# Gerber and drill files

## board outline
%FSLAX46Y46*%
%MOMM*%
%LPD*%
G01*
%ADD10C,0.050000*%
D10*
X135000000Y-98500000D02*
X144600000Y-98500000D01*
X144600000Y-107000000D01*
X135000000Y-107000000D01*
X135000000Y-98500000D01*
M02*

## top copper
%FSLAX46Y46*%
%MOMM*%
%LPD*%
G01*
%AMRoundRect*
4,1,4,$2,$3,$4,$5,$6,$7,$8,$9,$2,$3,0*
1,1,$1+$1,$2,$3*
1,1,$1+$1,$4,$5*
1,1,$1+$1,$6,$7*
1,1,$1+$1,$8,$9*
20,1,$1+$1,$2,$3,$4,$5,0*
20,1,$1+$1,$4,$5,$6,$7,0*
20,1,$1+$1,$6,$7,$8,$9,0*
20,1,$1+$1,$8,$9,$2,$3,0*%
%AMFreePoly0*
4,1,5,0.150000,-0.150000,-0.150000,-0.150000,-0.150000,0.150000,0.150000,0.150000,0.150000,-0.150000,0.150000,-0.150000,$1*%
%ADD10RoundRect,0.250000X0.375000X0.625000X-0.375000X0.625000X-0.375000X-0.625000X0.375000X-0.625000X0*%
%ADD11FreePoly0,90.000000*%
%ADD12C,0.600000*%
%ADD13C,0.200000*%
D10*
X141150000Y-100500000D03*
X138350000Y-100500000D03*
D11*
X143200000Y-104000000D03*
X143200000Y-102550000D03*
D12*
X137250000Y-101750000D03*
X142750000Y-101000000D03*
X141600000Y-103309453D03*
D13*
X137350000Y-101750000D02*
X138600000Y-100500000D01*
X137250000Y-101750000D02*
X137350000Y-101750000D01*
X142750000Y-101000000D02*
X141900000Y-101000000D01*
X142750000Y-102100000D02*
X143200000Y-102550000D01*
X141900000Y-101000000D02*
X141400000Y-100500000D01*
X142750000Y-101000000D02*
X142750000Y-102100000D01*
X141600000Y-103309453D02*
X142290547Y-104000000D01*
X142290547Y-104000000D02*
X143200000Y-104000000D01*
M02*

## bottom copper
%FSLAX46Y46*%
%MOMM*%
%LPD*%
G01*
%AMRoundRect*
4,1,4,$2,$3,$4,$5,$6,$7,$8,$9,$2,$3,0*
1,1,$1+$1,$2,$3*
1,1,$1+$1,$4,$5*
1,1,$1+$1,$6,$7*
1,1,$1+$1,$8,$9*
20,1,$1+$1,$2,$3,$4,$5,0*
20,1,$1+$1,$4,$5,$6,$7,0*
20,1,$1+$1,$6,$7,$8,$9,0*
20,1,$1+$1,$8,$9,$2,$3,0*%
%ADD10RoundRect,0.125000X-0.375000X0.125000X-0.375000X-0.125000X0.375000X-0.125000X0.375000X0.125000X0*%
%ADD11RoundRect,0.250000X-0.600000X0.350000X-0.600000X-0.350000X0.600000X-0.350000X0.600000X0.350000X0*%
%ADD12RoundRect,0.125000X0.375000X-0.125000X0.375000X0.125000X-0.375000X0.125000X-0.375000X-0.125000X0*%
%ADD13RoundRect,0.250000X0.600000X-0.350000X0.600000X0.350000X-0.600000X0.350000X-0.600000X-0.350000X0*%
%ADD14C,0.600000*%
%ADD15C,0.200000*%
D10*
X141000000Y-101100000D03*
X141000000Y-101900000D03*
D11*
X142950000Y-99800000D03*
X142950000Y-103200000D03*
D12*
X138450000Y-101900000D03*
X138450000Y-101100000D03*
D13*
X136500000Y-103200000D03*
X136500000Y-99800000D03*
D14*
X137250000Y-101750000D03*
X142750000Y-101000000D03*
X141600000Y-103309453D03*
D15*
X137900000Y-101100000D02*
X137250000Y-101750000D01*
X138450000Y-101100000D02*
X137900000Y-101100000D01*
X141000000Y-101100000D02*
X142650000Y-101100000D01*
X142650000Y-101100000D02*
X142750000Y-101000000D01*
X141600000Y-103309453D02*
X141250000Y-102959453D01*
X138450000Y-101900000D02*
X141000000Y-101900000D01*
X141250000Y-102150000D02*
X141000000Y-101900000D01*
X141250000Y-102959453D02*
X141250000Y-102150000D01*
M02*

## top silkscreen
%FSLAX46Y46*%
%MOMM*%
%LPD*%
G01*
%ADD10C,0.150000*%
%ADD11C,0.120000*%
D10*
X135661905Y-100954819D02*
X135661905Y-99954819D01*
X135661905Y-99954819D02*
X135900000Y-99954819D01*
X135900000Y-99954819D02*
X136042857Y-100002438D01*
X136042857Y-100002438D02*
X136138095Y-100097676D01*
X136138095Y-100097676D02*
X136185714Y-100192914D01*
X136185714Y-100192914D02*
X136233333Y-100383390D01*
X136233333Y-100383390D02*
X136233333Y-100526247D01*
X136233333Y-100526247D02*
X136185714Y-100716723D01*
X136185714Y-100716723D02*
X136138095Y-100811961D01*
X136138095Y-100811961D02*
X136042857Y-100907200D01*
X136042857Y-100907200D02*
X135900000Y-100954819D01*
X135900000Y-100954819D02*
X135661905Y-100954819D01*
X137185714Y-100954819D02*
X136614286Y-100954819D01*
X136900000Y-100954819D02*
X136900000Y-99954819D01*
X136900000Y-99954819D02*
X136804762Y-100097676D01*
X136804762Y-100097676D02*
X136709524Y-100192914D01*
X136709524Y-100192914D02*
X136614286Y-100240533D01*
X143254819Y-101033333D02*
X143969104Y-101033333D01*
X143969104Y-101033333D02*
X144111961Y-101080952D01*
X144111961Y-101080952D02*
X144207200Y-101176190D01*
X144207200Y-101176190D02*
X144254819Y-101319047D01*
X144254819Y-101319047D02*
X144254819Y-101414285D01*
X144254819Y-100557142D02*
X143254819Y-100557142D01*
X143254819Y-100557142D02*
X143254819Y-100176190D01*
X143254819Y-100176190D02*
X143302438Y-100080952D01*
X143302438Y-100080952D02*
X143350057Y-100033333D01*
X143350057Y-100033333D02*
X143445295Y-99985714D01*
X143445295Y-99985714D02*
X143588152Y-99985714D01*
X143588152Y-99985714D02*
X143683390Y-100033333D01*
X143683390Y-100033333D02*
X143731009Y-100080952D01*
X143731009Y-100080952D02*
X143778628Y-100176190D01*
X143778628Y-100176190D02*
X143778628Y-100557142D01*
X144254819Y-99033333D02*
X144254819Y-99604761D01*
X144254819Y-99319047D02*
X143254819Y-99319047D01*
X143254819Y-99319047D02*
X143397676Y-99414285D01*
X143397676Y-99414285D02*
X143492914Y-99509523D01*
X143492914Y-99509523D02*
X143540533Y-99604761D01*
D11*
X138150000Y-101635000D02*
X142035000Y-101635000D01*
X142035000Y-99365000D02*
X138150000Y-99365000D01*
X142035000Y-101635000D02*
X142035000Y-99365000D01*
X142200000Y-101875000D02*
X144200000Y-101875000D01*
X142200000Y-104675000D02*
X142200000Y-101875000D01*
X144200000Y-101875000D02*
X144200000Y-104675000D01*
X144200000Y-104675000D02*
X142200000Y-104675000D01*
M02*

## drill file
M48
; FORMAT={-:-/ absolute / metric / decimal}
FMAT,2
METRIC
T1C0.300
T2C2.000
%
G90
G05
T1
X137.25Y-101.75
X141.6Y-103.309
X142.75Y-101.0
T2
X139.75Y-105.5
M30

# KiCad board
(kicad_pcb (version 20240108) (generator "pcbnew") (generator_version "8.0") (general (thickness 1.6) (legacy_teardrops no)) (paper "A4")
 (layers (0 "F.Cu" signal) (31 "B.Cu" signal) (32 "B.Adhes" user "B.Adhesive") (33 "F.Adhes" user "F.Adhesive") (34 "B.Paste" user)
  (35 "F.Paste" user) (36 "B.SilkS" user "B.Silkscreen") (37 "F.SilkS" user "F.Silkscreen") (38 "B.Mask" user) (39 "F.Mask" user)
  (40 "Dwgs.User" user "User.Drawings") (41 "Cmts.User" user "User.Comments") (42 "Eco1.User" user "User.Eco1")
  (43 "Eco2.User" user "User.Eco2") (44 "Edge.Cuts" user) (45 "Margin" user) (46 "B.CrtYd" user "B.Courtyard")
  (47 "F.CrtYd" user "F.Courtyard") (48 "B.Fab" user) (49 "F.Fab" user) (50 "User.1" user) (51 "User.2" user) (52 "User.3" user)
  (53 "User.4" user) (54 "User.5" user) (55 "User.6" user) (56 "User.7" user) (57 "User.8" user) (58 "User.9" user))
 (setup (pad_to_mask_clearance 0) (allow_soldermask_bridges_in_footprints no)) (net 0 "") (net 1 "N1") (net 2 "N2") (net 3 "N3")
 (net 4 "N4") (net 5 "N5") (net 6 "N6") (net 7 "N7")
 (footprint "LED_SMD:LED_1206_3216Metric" (layer "F.Cu") (at 139.75 100.5 180)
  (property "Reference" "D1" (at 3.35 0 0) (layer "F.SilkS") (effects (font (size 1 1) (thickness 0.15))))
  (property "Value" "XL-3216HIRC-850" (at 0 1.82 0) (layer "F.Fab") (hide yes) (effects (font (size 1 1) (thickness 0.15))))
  (fp_line (start 1.6 -1.135) (end -2.285 -1.135) (stroke (width 0.12) (type solid)) (layer "F.SilkS"))
  (fp_line (start -2.285 1.135) (end 1.6 1.135) (stroke (width 0.12) (type solid)) (layer "F.SilkS"))
  (fp_line (start -2.285 -1.135) (end -2.285 1.135) (stroke (width 0.12) (type solid)) (layer "F.SilkS"))
  (pad "1" smd roundrect (at -1.4 0 180) (size 1.25 1.75) (layers "F.Cu" "F.Paste" "F.Mask") (roundrect_rratio 0.2) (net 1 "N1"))
  (pad "2" smd roundrect (at 1.4 0 180) (size 1.25 1.75) (layers "F.Cu" "F.Paste" "F.Mask") (roundrect_rratio 0.2) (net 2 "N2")))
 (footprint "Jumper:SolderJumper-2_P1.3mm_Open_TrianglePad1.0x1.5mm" (layer "F.Cu") (at 143.2 103.275 90)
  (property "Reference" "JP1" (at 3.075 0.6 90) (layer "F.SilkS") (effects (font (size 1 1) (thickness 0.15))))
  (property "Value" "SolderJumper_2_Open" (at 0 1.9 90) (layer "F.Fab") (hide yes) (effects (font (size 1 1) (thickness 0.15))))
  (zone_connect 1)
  (fp_line (start 1.4 -1) (end 1.4 1) (stroke (width 0.12) (type solid)) (layer "F.SilkS"))
  (fp_line (start -1.4 -1) (end 1.4 -1) (stroke (width 0.12) (type solid)) (layer "F.SilkS"))
  (fp_line (start 1.4 1) (end -1.4 1) (stroke (width 0.12) (type solid)) (layer "F.SilkS"))
  (fp_line (start -1.4 1) (end -1.4 -1) (stroke (width 0.12) (type solid)) (layer "F.SilkS"))
  (pad "1" smd custom (at -0.725 0 90) (size 0.3 0.3) (layers "F.Cu" "F.Mask") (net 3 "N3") (zone_connect 2) (thermal_bridge_angle 45)
   (options (clearance outline) (anchor rect)) (primitives))
  (pad "2" smd custom (at 0.725 0 90) (size 0.3 0.3) (layers "F.Cu" "F.Mask") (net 1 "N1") (zone_connect 2) (thermal_bridge_angle 45)
   (options (clearance outline) (anchor rect)) (primitives)))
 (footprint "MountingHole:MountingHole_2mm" (layer "F.Cu") (at 139.75 105.5)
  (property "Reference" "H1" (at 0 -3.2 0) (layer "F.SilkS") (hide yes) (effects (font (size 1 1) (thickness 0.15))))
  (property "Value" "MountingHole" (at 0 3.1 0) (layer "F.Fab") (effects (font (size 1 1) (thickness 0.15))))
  (pad "" np_thru_hole circle (at 0 0) (size 2 2) (drill 2) (layers "*.Cu" "*.Mask")))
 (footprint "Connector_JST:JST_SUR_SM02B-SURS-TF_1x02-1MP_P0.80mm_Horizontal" (layer "B.Cu") (at 142.15 101.5 -90)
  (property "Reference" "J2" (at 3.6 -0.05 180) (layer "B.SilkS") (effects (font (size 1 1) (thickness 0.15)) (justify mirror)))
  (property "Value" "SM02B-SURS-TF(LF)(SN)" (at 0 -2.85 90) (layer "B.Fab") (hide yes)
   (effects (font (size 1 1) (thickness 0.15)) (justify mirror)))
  (pad "1" smd roundrect (at -0.4 1.15 270) (size 0.5 1) (layers "B.Cu" "B.Paste" "B.Mask") (roundrect_rratio 0.25) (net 1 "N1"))
  (pad "2" smd roundrect (at 0.4 1.15 270) (size 0.5 1) (layers "B.Cu" "B.Paste" "B.Mask") (roundrect_rratio 0.25) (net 3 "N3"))
  (pad "MP" smd roundrect (at -1.7 -0.8 270) (size 1.2 1.7) (layers "B.Cu" "B.Paste" "B.Mask") (roundrect_rratio 0.208333) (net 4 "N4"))
  (pad "MP" smd roundrect (at 1.7 -0.8 270) (size 1.2 1.7) (layers "B.Cu" "B.Paste" "B.Mask") (roundrect_rratio 0.208333) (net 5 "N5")))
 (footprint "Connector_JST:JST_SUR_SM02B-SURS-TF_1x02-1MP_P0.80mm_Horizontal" (layer "B.Cu") (at 137.3 101.5 90)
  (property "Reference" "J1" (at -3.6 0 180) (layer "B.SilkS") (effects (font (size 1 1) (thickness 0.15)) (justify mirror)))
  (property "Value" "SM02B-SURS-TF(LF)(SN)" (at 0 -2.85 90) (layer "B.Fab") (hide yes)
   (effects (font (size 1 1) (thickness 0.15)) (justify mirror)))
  (pad "1" smd roundrect (at -0.4 1.15 90) (size 0.5 1) (layers "B.Cu" "B.Paste" "B.Mask") (roundrect_rratio 0.25) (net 3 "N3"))
  (pad "2" smd roundrect (at 0.4 1.15 90) (size 0.5 1) (layers "B.Cu" "B.Paste" "B.Mask") (roundrect_rratio 0.25) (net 2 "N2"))
  (pad "MP" smd roundrect (at -1.7 -0.8 90) (size 1.2 1.7) (layers "B.Cu" "B.Paste" "B.Mask") (roundrect_rratio 0.208333) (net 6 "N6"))
  (pad "MP" smd roundrect (at 1.7 -0.8 90) (size 1.2 1.7) (layers "B.Cu" "B.Paste" "B.Mask") (roundrect_rratio 0.208333) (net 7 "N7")))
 (gr_rect (start 135 98.5) (end 144.6 107) (stroke (width 0.05) (type default)) (fill none) (layer "Edge.Cuts"))
 (segment (start 137.35 101.75) (end 138.6 100.5) (width 0.2) (layer "F.Cu") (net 2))
 (segment (start 137.25 101.75) (end 137.35 101.75) (width 0.2) (layer "F.Cu") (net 2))
 (via (at 137.25 101.75) (size 0.6) (drill 0.3) (layers "F.Cu" "B.Cu") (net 2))
 (segment (start 137.9 101.1) (end 137.25 101.75) (width 0.2) (layer "B.Cu") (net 2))
 (segment (start 138.45 101.1) (end 137.9 101.1) (width 0.2) (layer "B.Cu") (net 2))
 (segment (start 142.75 101) (end 141.9 101) (width 0.2) (layer "F.Cu") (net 1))
 (segment (start 142.75 102.1) (end 143.2 102.55) (width 0.2) (layer "F.Cu") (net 1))
 (segment (start 141.9 101) (end 141.4 100.5) (width 0.2) (layer "F.Cu") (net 1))
 (segment (start 142.75 101) (end 142.75 102.1) (width 0.2) (layer "F.Cu") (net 1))
 (via (at 142.75 101) (size 0.6) (drill 0.3) (layers "F.Cu" "B.Cu") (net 1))
 (segment (start 141 101.1) (end 142.65 101.1) (width 0.2) (layer "B.Cu") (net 1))
 (segment (start 142.65 101.1) (end 142.75 101) (width 0.2) (layer "B.Cu") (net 1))
 (segment (start 141.6 103.309453) (end 142.290547 104) (width 0.2) (layer "F.Cu") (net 3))
 (segment (start 142.290547 104) (end 143.2 104) (width 0.2) (layer "F.Cu") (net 3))
 (via (at 141.6 103.309453) (size 0.6) (drill 0.3) (layers "F.Cu" "B.Cu") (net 3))
 (segment (start 141.6 103.309453) (end 141.25 102.959453) (width 0.2) (layer "B.Cu") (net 3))
 (segment (start 138.45 101.9) (end 141 101.9) (width 0.2) (layer "B.Cu") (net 3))
 (segment (start 141.25 102.15) (end 141 101.9) (width 0.2) (layer "B.Cu") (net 3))
 (segment (start 141.25 102.959453) (end 141.25 102.15) (width 0.2) (layer "B.Cu") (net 3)))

